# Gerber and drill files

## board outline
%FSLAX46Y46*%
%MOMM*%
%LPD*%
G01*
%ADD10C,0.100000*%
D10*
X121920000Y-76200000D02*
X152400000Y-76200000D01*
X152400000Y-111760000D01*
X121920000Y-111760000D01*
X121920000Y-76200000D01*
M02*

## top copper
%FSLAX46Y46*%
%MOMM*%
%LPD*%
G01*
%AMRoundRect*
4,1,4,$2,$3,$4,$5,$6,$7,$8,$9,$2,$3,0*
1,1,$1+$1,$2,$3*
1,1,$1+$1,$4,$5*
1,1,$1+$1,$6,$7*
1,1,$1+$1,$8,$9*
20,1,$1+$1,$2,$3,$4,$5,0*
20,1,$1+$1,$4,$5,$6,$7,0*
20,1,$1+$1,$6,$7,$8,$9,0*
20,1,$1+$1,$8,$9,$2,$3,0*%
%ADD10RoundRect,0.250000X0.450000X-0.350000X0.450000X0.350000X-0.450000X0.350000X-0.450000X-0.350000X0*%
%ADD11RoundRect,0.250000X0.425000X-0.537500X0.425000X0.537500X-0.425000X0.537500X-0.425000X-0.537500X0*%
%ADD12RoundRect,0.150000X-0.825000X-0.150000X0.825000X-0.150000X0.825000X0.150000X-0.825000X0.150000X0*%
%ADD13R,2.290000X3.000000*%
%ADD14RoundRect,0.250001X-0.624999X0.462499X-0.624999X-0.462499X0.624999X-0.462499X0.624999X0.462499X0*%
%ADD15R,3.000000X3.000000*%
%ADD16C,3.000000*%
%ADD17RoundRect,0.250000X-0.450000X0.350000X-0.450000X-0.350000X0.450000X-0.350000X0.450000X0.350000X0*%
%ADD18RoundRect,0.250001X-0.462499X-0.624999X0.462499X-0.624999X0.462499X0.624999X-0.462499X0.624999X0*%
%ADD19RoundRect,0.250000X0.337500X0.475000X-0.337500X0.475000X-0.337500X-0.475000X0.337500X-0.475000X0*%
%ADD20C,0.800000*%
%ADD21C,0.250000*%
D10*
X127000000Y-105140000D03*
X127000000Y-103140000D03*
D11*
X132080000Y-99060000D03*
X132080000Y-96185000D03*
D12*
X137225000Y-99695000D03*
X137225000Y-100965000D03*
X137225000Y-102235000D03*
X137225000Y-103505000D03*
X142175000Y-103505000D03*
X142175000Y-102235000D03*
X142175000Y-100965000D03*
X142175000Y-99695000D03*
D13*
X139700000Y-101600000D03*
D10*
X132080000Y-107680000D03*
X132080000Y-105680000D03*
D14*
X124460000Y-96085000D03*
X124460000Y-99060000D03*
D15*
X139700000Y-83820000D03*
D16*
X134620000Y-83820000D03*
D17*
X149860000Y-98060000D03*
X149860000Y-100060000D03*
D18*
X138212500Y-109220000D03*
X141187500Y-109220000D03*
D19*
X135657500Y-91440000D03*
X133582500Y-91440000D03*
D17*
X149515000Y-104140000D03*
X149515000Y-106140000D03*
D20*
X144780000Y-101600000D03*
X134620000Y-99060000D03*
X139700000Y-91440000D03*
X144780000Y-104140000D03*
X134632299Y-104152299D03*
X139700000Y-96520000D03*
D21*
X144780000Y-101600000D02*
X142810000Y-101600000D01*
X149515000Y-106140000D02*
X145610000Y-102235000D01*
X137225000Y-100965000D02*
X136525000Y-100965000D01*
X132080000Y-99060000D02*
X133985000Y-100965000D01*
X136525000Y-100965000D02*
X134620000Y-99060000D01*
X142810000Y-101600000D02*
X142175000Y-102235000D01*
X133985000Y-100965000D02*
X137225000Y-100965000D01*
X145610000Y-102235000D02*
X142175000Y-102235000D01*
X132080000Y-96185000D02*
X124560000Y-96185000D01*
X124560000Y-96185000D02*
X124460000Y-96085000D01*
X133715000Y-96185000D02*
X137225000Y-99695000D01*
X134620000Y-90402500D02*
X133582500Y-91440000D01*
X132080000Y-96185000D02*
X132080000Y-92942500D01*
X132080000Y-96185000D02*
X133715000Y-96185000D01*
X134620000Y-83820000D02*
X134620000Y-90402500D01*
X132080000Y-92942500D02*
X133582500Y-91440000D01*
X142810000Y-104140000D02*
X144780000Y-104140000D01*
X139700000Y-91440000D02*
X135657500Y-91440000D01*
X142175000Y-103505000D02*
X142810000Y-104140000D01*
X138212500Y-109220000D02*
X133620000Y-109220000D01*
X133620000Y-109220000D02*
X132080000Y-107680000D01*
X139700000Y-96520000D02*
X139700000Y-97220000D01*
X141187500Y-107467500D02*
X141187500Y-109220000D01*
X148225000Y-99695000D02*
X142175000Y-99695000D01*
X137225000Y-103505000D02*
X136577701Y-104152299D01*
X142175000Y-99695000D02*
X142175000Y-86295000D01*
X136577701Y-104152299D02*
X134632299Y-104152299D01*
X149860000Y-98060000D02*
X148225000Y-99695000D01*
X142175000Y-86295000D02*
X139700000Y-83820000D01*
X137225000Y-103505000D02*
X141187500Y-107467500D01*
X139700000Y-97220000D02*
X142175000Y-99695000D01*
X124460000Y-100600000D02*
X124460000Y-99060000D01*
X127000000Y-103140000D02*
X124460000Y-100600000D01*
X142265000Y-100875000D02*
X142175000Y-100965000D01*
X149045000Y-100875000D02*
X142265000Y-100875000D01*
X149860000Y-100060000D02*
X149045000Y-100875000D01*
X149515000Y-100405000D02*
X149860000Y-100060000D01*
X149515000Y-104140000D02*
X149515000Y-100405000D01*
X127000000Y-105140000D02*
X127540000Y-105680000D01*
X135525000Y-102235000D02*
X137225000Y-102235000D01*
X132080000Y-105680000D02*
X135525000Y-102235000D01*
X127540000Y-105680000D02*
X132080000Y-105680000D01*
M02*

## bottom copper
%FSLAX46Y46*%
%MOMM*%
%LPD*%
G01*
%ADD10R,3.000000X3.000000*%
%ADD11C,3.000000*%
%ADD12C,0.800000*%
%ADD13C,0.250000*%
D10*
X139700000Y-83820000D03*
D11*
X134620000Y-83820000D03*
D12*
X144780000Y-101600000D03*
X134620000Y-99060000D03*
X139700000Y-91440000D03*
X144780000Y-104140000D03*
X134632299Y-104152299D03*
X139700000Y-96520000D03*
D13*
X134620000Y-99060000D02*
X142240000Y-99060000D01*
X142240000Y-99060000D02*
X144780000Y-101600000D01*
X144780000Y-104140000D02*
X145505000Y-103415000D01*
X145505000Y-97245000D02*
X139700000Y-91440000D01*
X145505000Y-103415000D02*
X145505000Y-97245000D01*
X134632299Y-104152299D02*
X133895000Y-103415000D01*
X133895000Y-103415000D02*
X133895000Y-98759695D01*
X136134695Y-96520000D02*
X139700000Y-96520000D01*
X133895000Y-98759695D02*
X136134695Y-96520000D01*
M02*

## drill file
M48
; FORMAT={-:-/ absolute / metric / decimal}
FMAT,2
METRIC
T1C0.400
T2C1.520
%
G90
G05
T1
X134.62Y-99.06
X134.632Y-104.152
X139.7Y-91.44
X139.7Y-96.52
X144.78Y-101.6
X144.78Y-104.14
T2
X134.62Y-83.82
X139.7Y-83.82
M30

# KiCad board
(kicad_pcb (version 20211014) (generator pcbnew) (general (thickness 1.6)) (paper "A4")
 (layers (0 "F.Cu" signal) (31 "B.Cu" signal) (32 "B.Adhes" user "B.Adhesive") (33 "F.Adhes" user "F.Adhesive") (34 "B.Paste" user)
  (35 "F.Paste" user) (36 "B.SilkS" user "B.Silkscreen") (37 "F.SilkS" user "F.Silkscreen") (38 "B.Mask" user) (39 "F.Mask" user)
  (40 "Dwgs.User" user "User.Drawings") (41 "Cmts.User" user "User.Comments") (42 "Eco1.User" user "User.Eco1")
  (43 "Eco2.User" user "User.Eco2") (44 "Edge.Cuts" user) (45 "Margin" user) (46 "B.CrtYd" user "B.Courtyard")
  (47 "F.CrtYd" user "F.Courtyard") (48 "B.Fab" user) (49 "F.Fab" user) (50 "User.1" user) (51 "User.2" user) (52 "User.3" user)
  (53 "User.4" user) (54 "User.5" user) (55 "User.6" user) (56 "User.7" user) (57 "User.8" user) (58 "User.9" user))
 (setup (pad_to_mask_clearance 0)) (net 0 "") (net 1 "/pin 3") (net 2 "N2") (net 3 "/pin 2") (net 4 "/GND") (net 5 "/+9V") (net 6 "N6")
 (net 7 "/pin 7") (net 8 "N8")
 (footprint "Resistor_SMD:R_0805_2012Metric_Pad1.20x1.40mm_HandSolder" (layer "F.Cu") (at 127 104.14 90)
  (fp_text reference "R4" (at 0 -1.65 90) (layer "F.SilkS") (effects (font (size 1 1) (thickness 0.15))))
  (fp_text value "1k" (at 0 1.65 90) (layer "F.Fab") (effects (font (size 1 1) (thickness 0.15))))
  (pad "1" smd roundrect (at -1 0 90) (size 1.2 1.4) (layers "F.Cu" "F.Paste" "F.Mask") (roundrect_rratio 0.2083333333) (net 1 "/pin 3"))
  (pad "2" smd roundrect (at 1 0 90) (size 1.2 1.4) (layers "F.Cu" "F.Paste" "F.Mask") (roundrect_rratio 0.2083333333) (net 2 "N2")))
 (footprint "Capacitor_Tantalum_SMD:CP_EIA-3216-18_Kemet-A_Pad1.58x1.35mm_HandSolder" (layer "F.Cu") (at 132.08 97.6225 90)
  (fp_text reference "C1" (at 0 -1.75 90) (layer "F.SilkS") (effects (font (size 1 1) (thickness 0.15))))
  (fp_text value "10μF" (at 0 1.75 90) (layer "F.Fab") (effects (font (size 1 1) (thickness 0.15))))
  (pad "1" smd roundrect (at -1.4375 0 90) (size 1.575 1.35) (layers "F.Cu" "F.Paste" "F.Mask") (roundrect_rratio 0.1851851852)
   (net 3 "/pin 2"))
  (pad "2" smd roundrect (at 1.4375 0 90) (size 1.575 1.35) (layers "F.Cu" "F.Paste" "F.Mask") (roundrect_rratio 0.1851851852)
   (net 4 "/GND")))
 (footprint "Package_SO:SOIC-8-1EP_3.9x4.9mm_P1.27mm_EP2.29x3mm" (layer "F.Cu") (at 139.7 101.6)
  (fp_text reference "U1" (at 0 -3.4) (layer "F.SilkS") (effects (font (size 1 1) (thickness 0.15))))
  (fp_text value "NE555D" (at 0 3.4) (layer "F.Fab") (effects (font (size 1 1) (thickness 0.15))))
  (pad "" smd roundrect (at 0.57 0.75) (size 0.92 1.21) (layers "F.Paste") (roundrect_rratio 0.25))
  (pad "" smd roundrect (at -0.57 0.75) (size 0.92 1.21) (layers "F.Paste") (roundrect_rratio 0.25))
  (pad "" smd roundrect (at -0.57 -0.75) (size 0.92 1.21) (layers "F.Paste") (roundrect_rratio 0.25))
  (pad "" smd roundrect (at 0.57 -0.75) (size 0.92 1.21) (layers "F.Paste") (roundrect_rratio 0.25))
  (pad "1" smd roundrect (at -2.475 -1.905) (size 1.95 0.6) (layers "F.Cu" "F.Paste" "F.Mask") (roundrect_rratio 0.25) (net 4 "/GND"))
  (pad "2" smd roundrect (at -2.475 -0.635) (size 1.95 0.6) (layers "F.Cu" "F.Paste" "F.Mask") (roundrect_rratio 0.25) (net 3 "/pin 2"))
  (pad "3" smd roundrect (at -2.475 0.635) (size 1.95 0.6) (layers "F.Cu" "F.Paste" "F.Mask") (roundrect_rratio 0.25) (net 1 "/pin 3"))
  (pad "4" smd roundrect (at -2.475 1.905) (size 1.95 0.6) (layers "F.Cu" "F.Paste" "F.Mask") (roundrect_rratio 0.25) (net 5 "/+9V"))
  (pad "5" smd roundrect (at 2.475 1.905) (size 1.95 0.6) (layers "F.Cu" "F.Paste" "F.Mask") (roundrect_rratio 0.25) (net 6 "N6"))
  (pad "6" smd roundrect (at 2.475 0.635) (size 1.95 0.6) (layers "F.Cu" "F.Paste" "F.Mask") (roundrect_rratio 0.25) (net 3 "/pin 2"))
  (pad "7" smd roundrect (at 2.475 -0.635) (size 1.95 0.6) (layers "F.Cu" "F.Paste" "F.Mask") (roundrect_rratio 0.25) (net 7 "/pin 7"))
  (pad "8" smd roundrect (at 2.475 -1.905) (size 1.95 0.6) (layers "F.Cu" "F.Paste" "F.Mask") (roundrect_rratio 0.25) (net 5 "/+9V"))
  (pad "9" smd rect (at 0 0) (size 2.29 3) (layers "F.Cu" "F.Mask")))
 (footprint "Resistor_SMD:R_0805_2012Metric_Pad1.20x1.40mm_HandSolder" (layer "F.Cu") (at 132.08 106.68 90)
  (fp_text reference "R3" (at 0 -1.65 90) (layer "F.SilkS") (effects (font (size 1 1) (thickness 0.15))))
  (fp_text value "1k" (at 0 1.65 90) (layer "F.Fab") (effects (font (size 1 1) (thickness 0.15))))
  (pad "1" smd roundrect (at -1 0 90) (size 1.2 1.4) (layers "F.Cu" "F.Paste" "F.Mask") (roundrect_rratio 0.2083333333) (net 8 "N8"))
  (pad "2" smd roundrect (at 1 0 90) (size 1.2 1.4) (layers "F.Cu" "F.Paste" "F.Mask") (roundrect_rratio 0.2083333333) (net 1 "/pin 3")))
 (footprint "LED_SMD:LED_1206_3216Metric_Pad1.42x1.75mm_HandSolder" (layer "F.Cu") (at 124.46 97.5725 -90)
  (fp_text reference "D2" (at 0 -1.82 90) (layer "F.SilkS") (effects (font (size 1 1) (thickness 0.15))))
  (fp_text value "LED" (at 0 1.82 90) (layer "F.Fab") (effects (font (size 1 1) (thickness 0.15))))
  (pad "1" smd roundrect (at -1.4875 0 270) (size 1.425 1.75) (layers "F.Cu" "F.Paste" "F.Mask") (roundrect_rratio 0.1754392982)
   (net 4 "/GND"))
  (pad "2" smd roundrect (at 1.4875 0 270) (size 1.425 1.75) (layers "F.Cu" "F.Paste" "F.Mask") (roundrect_rratio 0.1754392982) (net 2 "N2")))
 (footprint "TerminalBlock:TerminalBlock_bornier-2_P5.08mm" (layer "F.Cu") (at 139.7 83.82 180)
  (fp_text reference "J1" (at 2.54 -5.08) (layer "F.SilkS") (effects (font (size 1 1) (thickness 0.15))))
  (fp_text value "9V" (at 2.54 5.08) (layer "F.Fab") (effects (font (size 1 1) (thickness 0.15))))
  (pad "1" thru_hole rect (at 0 0 180) (size 3 3) (drill 1.52) (layers *.Cu *.Mask) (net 5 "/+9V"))
  (pad "2" thru_hole circle (at 5.08 0 180) (size 3 3) (drill 1.52) (layers *.Cu *.Mask) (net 4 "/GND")))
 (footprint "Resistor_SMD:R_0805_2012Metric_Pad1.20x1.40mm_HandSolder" (layer "F.Cu") (at 149.86 99.06 -90)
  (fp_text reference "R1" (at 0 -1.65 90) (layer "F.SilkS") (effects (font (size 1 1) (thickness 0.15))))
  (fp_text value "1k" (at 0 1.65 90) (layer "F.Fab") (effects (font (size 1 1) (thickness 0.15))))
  (pad "1" smd roundrect (at -1 0 270) (size 1.2 1.4) (layers "F.Cu" "F.Paste" "F.Mask") (roundrect_rratio 0.2083333333) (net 5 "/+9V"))
  (pad "2" smd roundrect (at 1 0 270) (size 1.2 1.4) (layers "F.Cu" "F.Paste" "F.Mask") (roundrect_rratio 0.2083333333) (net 7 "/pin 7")))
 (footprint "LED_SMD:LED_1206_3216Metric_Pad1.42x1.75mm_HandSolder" (layer "F.Cu") (at 139.7 109.22)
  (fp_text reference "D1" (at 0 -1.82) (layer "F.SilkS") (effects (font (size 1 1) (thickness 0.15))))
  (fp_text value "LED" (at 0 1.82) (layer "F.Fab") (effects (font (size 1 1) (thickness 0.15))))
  (pad "1" smd roundrect (at -1.4875 0) (size 1.425 1.75) (layers "F.Cu" "F.Paste" "F.Mask") (roundrect_rratio 0.1754392982) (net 8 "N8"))
  (pad "2" smd roundrect (at 1.4875 0) (size 1.425 1.75) (layers "F.Cu" "F.Paste" "F.Mask") (roundrect_rratio 0.1754392982) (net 5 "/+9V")))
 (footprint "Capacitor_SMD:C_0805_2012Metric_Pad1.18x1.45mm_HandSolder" (layer "F.Cu") (at 134.62 91.44 180)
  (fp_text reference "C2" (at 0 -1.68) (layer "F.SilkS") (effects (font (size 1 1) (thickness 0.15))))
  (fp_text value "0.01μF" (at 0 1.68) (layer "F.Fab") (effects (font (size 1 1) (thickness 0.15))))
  (pad "1" smd roundrect (at -1.0375 0 180) (size 1.175 1.45) (layers "F.Cu" "F.Paste" "F.Mask") (roundrect_rratio 0.2127659574)
   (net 6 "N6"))
  (pad "2" smd roundrect (at 1.0375 0 180) (size 1.175 1.45) (layers "F.Cu" "F.Paste" "F.Mask") (roundrect_rratio 0.2127659574)
   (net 4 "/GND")))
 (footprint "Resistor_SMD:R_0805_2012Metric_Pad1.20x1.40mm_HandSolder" (layer "F.Cu") (at 149.515 105.14 -90)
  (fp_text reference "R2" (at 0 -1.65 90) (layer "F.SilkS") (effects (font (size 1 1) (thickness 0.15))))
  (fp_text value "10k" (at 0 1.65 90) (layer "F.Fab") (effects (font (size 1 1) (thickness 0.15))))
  (pad "1" smd roundrect (at -1 0 270) (size 1.2 1.4) (layers "F.Cu" "F.Paste" "F.Mask") (roundrect_rratio 0.2083333333) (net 7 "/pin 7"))
  (pad "2" smd roundrect (at 1 0 270) (size 1.2 1.4) (layers "F.Cu" "F.Paste" "F.Mask") (roundrect_rratio 0.2083333333) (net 3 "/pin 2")))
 (gr_rect (start 121.92 76.2) (end 152.4 111.76) (layer "Edge.Cuts") (width 0.1) (fill none))
 (segment (start 144.78 101.6) (end 142.81 101.6) (width 0.25) (layer "F.Cu") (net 3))
 (segment (start 149.515 106.14) (end 145.61 102.235) (width 0.25) (layer "F.Cu") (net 3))
 (segment (start 137.225 100.965) (end 136.525 100.965) (width 0.25) (layer "F.Cu") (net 3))
 (segment (start 132.08 99.06) (end 133.985 100.965) (width 0.25) (layer "F.Cu") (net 3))
 (segment (start 136.525 100.965) (end 134.62 99.06) (width 0.25) (layer "F.Cu") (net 3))
 (segment (start 142.81 101.6) (end 142.175 102.235) (width 0.25) (layer "F.Cu") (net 3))
 (segment (start 133.985 100.965) (end 137.225 100.965) (width 0.25) (layer "F.Cu") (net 3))
 (segment (start 145.61 102.235) (end 142.175 102.235) (width 0.25) (layer "F.Cu") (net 3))
 (via (at 144.78 101.6) (size 0.8) (drill 0.4) (layers "F.Cu" "B.Cu") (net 3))
 (via (at 134.62 99.06) (size 0.8) (drill 0.4) (layers "F.Cu" "B.Cu") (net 3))
 (segment (start 134.62 99.06) (end 142.24 99.06) (width 0.25) (layer "B.Cu") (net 3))
 (segment (start 142.24 99.06) (end 144.78 101.6) (width 0.25) (layer "B.Cu") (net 3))
 (segment (start 132.08 96.185) (end 124.56 96.185) (width 0.25) (layer "F.Cu") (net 4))
 (segment (start 124.56 96.185) (end 124.46 96.085) (width 0.25) (layer "F.Cu") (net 4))
 (segment (start 133.715 96.185) (end 137.225 99.695) (width 0.25) (layer "F.Cu") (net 4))
 (segment (start 134.62 90.4025) (end 133.5825 91.44) (width 0.25) (layer "F.Cu") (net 4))
 (segment (start 132.08 96.185) (end 132.08 92.9425) (width 0.25) (layer "F.Cu") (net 4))
 (segment (start 132.08 96.185) (end 133.715 96.185) (width 0.25) (layer "F.Cu") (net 4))
 (segment (start 134.62 83.82) (end 134.62 90.4025) (width 0.25) (layer "F.Cu") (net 4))
 (segment (start 132.08 92.9425) (end 133.5825 91.44) (width 0.25) (layer "F.Cu") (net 4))
 (segment (start 142.81 104.14) (end 144.78 104.14) (width 0.25) (layer "F.Cu") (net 6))
 (segment (start 139.7 91.44) (end 135.6575 91.44) (width 0.25) (layer "F.Cu") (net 6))
 (segment (start 142.175 103.505) (end 142.81 104.14) (width 0.25) (layer "F.Cu") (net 6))
 (via (at 139.7 91.44) (size 0.8) (drill 0.4) (layers "F.Cu" "B.Cu") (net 6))
 (via (at 144.78 104.14) (size 0.8) (drill 0.4) (layers "F.Cu" "B.Cu") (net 6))
 (segment (start 144.78 104.14) (end 145.505 103.415) (width 0.25) (layer "B.Cu") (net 6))
 (segment (start 145.505 97.245) (end 139.7 91.44) (width 0.25) (layer "B.Cu") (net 6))
 (segment (start 145.505 103.415) (end 145.505 97.245) (width 0.25) (layer "B.Cu") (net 6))
 (segment (start 138.2125 109.22) (end 133.62 109.22) (width 0.25) (layer "F.Cu") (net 8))
 (segment (start 133.62 109.22) (end 132.08 107.68) (width 0.25) (layer "F.Cu") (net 8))
 (segment (start 139.7 96.52) (end 139.7 97.22) (width 0.25) (layer "F.Cu") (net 5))
 (segment (start 141.1875 107.4675) (end 141.1875 109.22) (width 0.25) (layer "F.Cu") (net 5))
 (segment (start 148.225 99.695) (end 142.175 99.695) (width 0.25) (layer "F.Cu") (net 5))
 (segment (start 137.225 103.505) (end 136.577701 104.152299) (width 0.25) (layer "F.Cu") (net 5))
 (segment (start 142.175 99.695) (end 142.175 86.295) (width 0.25) (layer "F.Cu") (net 5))
 (segment (start 136.577701 104.152299) (end 134.632299 104.152299) (width 0.25) (layer "F.Cu") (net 5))
 (segment (start 149.86 98.06) (end 148.225 99.695) (width 0.25) (layer "F.Cu") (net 5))
 (segment (start 142.175 86.295) (end 139.7 83.82) (width 0.25) (layer "F.Cu") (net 5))
 (segment (start 137.225 103.505) (end 141.1875 107.4675) (width 0.25) (layer "F.Cu") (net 5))
 (segment (start 139.7 97.22) (end 142.175 99.695) (width 0.25) (layer "F.Cu") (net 5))
 (via (at 134.632299 104.152299) (size 0.8) (drill 0.4) (layers "F.Cu" "B.Cu") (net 5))
 (via (at 139.7 96.52) (size 0.8) (drill 0.4) (layers "F.Cu" "B.Cu") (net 5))
 (segment (start 134.632299 104.152299) (end 133.895 103.415) (width 0.25) (layer "B.Cu") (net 5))
 (segment (start 133.895 103.415) (end 133.895 98.759695) (width 0.25) (layer "B.Cu") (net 5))
 (segment (start 136.134695 96.52) (end 139.7 96.52) (width 0.25) (layer "B.Cu") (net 5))
 (segment (start 133.895 98.759695) (end 136.134695 96.52) (width 0.25) (layer "B.Cu") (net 5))
 (segment (start 124.46 100.6) (end 124.46 99.06) (width 0.25) (layer "F.Cu") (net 2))
 (segment (start 127 103.14) (end 124.46 100.6) (width 0.25) (layer "F.Cu") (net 2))
 (segment (start 142.265 100.875) (end 142.175 100.965) (width 0.25) (layer "F.Cu") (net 7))
 (segment (start 149.045 100.875) (end 142.265 100.875) (width 0.25) (layer "F.Cu") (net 7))
 (segment (start 149.86 100.06) (end 149.045 100.875) (width 0.25) (layer "F.Cu") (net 7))
 (segment (start 149.515 100.405) (end 149.86 100.06) (width 0.25) (layer "F.Cu") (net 7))
 (segment (start 149.515 104.14) (end 149.515 100.405) (width 0.25) (layer "F.Cu") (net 7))
 (segment (start 127 105.14) (end 127.54 105.68) (width 0.25) (layer "F.Cu") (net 1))
 (segment (start 135.525 102.235) (end 137.225 102.235) (width 0.25) (layer "F.Cu") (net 1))
 (segment (start 132.08 105.68) (end 135.525 102.235) (width 0.25) (layer "F.Cu") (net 1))
 (segment (start 127.54 105.68) (end 132.08 105.68) (width 0.25) (layer "F.Cu") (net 1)))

